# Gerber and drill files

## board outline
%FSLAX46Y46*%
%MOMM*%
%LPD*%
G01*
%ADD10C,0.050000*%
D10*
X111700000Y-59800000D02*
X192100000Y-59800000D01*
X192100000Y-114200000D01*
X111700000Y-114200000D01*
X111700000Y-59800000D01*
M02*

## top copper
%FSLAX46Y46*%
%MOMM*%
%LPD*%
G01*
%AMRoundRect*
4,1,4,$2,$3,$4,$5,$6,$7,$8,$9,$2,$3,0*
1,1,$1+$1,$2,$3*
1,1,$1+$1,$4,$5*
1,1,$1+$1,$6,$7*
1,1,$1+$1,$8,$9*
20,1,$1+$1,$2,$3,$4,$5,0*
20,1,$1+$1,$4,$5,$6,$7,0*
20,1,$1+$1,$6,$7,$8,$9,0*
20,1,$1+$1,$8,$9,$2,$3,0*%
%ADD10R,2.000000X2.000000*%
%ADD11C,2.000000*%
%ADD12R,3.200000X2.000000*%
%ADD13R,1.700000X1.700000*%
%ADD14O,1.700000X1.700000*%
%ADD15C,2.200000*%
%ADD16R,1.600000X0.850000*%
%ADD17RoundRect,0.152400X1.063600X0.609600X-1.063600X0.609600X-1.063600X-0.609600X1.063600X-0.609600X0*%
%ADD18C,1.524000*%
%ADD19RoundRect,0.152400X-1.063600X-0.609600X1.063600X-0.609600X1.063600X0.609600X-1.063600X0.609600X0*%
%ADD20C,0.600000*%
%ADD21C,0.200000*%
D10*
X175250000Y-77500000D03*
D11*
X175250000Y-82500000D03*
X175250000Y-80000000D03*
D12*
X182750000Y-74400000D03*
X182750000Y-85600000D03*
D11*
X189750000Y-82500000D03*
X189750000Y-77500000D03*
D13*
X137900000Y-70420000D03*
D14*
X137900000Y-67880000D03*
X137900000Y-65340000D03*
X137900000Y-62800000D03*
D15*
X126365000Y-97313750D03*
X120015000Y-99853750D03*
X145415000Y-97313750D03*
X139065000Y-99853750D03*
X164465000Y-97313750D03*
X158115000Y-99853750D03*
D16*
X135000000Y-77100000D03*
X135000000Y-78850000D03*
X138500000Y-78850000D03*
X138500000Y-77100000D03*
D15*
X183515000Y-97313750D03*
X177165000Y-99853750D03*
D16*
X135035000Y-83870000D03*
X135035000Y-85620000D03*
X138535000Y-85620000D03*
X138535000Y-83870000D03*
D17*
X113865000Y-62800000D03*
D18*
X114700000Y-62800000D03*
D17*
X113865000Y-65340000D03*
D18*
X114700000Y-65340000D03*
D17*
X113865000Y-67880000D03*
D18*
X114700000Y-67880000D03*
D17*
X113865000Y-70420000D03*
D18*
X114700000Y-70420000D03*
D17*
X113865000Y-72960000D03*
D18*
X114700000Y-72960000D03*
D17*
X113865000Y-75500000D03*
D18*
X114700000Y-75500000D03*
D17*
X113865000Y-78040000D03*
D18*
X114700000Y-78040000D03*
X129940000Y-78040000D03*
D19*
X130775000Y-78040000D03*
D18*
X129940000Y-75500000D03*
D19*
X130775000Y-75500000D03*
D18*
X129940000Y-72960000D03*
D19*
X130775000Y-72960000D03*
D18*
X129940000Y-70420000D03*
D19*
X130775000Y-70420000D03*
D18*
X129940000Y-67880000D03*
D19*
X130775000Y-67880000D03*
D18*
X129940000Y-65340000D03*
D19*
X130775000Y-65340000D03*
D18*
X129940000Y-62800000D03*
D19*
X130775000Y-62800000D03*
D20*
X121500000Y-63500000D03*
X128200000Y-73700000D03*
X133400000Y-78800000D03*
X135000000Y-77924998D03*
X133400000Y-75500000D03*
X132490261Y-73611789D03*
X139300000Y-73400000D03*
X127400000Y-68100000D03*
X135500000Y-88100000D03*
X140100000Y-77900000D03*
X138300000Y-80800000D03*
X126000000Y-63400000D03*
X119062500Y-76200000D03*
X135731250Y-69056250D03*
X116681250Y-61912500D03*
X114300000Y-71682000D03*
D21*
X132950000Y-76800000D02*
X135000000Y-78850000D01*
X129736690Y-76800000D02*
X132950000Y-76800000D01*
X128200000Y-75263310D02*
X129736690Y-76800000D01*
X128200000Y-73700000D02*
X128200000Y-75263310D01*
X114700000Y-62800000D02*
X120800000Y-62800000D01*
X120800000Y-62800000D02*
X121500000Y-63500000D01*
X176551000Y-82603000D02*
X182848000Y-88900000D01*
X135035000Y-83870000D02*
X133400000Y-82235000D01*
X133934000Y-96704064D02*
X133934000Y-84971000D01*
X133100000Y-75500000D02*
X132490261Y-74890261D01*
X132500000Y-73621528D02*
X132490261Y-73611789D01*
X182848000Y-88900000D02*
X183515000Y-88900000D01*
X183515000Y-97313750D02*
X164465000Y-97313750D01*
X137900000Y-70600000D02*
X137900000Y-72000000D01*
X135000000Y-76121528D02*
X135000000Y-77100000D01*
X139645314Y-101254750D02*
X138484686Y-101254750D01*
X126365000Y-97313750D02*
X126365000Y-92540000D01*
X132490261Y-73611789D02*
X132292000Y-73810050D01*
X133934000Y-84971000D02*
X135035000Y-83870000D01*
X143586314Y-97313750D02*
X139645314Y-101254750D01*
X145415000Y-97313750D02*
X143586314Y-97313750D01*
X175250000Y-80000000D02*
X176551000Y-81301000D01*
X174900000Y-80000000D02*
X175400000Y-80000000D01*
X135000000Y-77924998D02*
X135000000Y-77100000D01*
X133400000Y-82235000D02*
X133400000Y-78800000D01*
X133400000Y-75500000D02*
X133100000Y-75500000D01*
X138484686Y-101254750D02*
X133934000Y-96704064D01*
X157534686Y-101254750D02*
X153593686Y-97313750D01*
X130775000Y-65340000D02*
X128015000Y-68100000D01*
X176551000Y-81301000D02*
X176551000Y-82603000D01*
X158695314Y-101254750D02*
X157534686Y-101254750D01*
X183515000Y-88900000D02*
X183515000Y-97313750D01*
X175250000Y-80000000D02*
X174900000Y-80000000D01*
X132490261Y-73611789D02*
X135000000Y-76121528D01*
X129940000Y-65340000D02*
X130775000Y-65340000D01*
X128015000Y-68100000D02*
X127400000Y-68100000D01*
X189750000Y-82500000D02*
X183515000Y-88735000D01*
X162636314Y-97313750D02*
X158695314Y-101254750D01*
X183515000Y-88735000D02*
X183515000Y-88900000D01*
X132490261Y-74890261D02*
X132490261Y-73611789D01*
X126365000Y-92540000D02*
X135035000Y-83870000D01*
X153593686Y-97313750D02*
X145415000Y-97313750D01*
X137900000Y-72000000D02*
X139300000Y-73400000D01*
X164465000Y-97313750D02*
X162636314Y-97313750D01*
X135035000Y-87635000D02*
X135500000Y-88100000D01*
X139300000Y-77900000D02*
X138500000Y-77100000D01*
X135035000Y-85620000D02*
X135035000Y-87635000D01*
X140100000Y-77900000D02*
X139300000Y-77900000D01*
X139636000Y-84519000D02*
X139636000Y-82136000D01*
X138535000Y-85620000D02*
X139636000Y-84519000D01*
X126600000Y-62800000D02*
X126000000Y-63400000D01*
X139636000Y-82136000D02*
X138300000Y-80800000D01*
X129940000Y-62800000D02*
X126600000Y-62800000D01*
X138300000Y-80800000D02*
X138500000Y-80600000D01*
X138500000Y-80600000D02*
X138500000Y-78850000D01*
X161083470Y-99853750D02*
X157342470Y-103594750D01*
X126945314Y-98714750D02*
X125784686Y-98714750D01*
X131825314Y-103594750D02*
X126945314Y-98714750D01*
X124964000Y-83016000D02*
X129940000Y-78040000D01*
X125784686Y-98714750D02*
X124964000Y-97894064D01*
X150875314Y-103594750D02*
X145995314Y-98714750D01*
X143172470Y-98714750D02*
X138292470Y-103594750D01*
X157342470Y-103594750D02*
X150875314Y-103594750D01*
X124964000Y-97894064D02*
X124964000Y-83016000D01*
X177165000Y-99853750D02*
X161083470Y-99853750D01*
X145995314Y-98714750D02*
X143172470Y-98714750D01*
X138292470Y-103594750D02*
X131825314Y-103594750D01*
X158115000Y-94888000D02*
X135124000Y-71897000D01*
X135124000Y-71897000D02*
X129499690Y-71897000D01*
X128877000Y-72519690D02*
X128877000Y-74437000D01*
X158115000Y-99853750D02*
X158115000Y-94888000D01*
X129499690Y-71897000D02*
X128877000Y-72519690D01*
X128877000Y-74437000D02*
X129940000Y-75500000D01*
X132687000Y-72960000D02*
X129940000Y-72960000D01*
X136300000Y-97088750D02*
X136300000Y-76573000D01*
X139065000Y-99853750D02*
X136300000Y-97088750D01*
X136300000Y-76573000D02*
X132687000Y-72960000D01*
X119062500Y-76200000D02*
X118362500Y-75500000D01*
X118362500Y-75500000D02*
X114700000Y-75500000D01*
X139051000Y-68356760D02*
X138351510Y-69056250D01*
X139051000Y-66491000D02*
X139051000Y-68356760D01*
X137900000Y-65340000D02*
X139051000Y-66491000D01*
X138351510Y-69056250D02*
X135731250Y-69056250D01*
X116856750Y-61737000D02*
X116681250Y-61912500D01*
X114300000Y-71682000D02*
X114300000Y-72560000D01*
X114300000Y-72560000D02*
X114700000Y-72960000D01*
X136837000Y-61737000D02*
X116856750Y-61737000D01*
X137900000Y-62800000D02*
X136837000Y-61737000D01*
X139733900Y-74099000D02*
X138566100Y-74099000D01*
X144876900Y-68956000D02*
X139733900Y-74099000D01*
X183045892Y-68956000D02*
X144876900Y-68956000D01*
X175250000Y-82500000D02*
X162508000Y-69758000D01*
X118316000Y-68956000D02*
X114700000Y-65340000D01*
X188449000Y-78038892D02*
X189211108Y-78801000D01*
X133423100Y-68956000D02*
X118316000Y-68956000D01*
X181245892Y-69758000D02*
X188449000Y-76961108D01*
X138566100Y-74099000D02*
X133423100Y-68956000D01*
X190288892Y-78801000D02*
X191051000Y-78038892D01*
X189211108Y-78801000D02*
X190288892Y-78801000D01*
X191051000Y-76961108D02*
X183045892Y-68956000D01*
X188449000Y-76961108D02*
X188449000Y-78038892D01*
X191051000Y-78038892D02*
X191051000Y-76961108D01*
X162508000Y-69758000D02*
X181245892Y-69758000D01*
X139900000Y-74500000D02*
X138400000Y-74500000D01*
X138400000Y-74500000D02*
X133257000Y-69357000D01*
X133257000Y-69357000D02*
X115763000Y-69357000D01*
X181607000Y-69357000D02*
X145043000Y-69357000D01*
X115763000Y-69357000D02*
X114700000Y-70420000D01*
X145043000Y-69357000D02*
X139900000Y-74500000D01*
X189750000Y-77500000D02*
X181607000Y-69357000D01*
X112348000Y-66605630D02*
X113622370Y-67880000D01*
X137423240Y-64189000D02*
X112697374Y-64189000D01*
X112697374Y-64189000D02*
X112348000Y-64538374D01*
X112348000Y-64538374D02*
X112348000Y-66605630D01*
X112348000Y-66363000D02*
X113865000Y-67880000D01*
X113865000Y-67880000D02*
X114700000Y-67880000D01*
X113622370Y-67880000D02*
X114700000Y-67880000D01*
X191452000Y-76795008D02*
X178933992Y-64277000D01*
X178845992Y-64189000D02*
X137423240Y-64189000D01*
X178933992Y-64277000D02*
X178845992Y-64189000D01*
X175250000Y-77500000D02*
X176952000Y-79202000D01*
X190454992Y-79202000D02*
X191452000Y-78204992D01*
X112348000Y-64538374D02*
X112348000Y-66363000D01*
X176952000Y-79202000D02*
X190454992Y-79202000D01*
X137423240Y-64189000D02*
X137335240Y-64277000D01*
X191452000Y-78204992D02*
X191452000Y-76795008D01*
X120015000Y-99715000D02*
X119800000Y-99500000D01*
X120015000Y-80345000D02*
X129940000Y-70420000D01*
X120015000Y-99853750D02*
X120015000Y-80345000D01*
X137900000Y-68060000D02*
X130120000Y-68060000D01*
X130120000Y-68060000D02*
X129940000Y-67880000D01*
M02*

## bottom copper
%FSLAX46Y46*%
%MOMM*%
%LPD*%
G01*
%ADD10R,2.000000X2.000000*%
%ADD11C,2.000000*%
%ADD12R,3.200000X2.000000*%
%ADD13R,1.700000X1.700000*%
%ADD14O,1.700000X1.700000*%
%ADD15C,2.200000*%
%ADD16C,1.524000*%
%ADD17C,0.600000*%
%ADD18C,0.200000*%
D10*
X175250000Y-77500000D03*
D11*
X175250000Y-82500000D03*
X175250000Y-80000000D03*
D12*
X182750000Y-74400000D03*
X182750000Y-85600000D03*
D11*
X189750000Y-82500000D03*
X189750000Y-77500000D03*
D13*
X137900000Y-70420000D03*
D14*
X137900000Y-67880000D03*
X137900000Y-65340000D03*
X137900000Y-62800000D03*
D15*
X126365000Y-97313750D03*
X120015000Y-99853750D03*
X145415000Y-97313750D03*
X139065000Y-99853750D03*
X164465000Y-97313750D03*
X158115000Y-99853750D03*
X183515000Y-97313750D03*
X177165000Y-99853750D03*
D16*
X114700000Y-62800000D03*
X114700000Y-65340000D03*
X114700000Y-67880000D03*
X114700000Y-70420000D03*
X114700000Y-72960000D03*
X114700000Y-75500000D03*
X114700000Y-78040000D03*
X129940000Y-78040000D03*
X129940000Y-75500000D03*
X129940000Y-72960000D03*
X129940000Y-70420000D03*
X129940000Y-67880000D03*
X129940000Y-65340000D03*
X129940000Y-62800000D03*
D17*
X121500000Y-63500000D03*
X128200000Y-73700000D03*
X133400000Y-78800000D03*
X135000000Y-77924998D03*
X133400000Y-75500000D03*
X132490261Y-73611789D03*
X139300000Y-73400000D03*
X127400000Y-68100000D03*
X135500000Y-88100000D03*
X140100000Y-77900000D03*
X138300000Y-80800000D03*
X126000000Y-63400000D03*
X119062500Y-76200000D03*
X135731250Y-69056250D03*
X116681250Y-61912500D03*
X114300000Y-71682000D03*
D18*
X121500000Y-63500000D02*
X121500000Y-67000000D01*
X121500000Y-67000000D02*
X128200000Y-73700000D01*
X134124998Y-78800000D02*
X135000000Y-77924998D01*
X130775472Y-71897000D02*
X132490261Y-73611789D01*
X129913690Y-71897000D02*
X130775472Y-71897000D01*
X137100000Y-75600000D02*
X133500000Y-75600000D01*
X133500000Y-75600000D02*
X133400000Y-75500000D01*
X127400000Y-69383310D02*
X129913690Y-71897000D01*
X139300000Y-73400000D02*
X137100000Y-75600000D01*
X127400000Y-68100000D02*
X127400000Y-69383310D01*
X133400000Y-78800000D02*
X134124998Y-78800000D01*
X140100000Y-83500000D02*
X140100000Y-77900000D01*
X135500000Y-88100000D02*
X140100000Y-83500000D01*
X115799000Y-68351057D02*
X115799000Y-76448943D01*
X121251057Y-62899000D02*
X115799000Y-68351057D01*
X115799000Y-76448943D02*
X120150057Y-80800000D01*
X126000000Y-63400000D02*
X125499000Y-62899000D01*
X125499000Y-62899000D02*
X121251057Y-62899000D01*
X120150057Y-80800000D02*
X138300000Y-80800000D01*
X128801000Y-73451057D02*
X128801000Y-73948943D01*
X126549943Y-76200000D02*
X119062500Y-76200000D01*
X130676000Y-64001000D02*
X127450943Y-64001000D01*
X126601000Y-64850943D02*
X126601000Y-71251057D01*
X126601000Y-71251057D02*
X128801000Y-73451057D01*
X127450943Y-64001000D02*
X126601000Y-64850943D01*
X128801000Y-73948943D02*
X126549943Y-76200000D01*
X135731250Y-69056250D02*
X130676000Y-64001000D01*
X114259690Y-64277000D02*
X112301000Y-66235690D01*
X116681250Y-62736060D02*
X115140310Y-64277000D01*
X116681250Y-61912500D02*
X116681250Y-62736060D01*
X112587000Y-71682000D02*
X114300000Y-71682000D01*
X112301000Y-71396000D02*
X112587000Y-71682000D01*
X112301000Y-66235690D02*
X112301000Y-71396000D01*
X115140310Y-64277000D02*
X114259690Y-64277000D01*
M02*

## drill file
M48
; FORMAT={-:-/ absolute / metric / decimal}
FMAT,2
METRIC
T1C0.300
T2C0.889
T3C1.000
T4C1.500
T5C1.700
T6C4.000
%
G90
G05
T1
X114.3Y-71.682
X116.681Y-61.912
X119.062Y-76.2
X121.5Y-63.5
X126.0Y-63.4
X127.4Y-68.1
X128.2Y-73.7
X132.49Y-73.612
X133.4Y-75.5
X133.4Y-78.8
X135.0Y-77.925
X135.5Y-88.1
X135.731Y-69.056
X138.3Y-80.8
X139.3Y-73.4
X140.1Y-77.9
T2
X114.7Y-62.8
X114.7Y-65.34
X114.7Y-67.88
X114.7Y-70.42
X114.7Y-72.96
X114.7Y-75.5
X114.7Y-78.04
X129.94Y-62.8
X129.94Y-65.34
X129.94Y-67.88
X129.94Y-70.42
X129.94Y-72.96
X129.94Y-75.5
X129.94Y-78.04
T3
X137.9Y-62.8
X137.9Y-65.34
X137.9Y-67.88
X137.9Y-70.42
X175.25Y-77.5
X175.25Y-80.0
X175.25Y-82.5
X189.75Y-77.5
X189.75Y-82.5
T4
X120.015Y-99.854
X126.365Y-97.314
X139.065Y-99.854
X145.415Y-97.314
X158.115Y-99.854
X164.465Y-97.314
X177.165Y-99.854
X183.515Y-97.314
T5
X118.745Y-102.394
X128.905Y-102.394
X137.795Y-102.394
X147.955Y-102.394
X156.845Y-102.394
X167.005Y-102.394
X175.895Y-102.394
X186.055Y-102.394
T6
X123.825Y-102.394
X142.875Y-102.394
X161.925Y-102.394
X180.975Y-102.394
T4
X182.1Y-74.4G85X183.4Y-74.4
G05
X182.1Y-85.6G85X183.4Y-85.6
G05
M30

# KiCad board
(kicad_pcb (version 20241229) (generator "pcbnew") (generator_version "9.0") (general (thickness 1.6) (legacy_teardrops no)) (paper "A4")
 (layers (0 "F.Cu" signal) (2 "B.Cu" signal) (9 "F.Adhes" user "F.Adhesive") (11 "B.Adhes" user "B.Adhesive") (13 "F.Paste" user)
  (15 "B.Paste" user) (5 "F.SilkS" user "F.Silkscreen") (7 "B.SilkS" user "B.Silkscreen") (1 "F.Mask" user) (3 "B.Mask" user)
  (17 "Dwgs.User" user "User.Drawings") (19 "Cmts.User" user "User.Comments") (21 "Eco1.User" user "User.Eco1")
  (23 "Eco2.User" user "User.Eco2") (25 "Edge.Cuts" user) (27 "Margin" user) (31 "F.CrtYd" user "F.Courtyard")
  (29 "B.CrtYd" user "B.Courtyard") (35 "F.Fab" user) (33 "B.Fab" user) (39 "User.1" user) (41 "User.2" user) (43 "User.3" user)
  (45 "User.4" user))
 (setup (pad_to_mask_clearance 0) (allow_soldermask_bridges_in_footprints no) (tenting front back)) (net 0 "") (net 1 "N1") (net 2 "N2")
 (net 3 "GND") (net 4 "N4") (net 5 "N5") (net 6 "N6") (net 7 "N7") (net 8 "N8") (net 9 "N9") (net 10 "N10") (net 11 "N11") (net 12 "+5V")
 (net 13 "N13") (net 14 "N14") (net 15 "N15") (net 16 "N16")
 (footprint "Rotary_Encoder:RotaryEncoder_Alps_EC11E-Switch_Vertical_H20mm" (layer "F.Cu") (at 175.25 77.5)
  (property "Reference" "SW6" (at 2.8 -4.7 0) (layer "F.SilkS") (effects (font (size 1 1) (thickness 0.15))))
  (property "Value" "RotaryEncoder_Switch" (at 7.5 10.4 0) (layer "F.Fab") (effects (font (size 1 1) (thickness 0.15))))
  (pad "A" thru_hole rect (at 0 0) (size 2 2) (drill 1) (layers "*.Cu" "*.Mask") (remove_unused_layers no) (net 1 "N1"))
  (pad "B" thru_hole circle (at 0 5) (size 2 2) (drill 1) (layers "*.Cu" "*.Mask") (remove_unused_layers no) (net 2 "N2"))
  (pad "C" thru_hole circle (at 0 2.5) (size 2 2) (drill 1) (layers "*.Cu" "*.Mask") (remove_unused_layers no) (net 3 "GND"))
  (pad "MP" thru_hole rect (at 7.5 -3.1) (size 3.2 2) (drill oval 2.8 1.5) (layers "*.Cu" "*.Mask") (remove_unused_layers no))
  (pad "MP" thru_hole rect (at 7.5 8.1) (size 3.2 2) (drill oval 2.8 1.5) (layers "*.Cu" "*.Mask") (remove_unused_layers no))
  (pad "S1" thru_hole circle (at 14.5 5) (size 2 2) (drill 1) (layers "*.Cu" "*.Mask") (remove_unused_layers no) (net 3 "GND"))
  (pad "S2" thru_hole circle (at 14.5 0) (size 2 2) (drill 1) (layers "*.Cu" "*.Mask") (remove_unused_layers no) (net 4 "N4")))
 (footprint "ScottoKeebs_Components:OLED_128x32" (layer "F.Cu") (at 136.3 60.62)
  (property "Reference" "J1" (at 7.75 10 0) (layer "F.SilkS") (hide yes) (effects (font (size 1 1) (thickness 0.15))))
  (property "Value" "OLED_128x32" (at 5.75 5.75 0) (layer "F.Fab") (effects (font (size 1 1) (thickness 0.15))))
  (pad "1" thru_hole rect (at 1.6 9.8 180) (size 1.7 1.7) (drill 1) (layers "*.Cu" "*.Mask") (remove_unused_layers no) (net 3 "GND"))
  (pad "2" thru_hole oval (at 1.6 7.26 180) (size 1.7 1.7) (drill 1) (layers "*.Cu" "*.Mask") (remove_unused_layers no) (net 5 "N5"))
  (pad "3" thru_hole oval (at 1.6 4.72 180) (size 1.7 1.7) (drill 1) (layers "*.Cu" "*.Mask") (remove_unused_layers no) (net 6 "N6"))
  (pad "4" thru_hole oval (at 1.6 2.18 180) (size 1.7 1.7) (drill 1) (layers "*.Cu" "*.Mask") (remove_unused_layers no) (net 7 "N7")))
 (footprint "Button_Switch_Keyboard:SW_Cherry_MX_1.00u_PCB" (layer "F.Cu") (at 126.365 97.31375)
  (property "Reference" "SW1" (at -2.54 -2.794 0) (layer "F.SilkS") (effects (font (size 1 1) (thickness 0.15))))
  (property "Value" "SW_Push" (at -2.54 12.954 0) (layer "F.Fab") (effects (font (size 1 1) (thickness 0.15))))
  (pad "" np_thru_hole circle (at -7.62 5.08) (size 1.7 1.7) (drill 1.7) (layers "*.Cu" "*.Mask"))
  (pad "" np_thru_hole circle (at -2.54 5.08) (size 4 4) (drill 4) (layers "*.Cu" "*.Mask"))
  (pad "" np_thru_hole circle (at 2.54 5.08) (size 1.7 1.7) (drill 1.7) (layers "*.Cu" "*.Mask"))
  (pad "1" thru_hole circle (at 0 0) (size 2.2 2.2) (drill 1.5) (layers "*.Cu" "*.Mask") (remove_unused_layers no) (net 3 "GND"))
  (pad "2" thru_hole circle (at -6.35 2.54) (size 2.2 2.2) (drill 1.5) (layers "*.Cu" "*.Mask") (remove_unused_layers no) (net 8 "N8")))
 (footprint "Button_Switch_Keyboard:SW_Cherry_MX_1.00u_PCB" (layer "F.Cu") (at 145.415 97.31375)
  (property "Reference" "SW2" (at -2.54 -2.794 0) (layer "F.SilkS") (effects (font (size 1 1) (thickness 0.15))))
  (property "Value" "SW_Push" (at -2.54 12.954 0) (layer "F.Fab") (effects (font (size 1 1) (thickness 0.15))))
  (pad "" np_thru_hole circle (at -7.62 5.08) (size 1.7 1.7) (drill 1.7) (layers "*.Cu" "*.Mask"))
  (pad "" np_thru_hole circle (at -2.54 5.08) (size 4 4) (drill 4) (layers "*.Cu" "*.Mask"))
  (pad "" np_thru_hole circle (at 2.54 5.08) (size 1.7 1.7) (drill 1.7) (layers "*.Cu" "*.Mask"))
  (pad "1" thru_hole circle (at 0 0) (size 2.2 2.2) (drill 1.5) (layers "*.Cu" "*.Mask") (remove_unused_layers no) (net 3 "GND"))
  (pad "2" thru_hole circle (at -6.35 2.54) (size 2.2 2.2) (drill 1.5) (layers "*.Cu" "*.Mask") (remove_unused_layers no) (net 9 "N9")))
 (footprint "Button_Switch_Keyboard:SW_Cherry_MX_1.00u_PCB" (layer "F.Cu") (at 164.465 97.31375)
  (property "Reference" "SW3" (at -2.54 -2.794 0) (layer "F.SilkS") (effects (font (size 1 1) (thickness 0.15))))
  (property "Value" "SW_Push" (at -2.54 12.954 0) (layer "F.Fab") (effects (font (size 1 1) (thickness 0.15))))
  (pad "" np_thru_hole circle (at -7.62 5.08) (size 1.7 1.7) (drill 1.7) (layers "*.Cu" "*.Mask"))
  (pad "" np_thru_hole circle (at -2.54 5.08) (size 4 4) (drill 4) (layers "*.Cu" "*.Mask"))
  (pad "" np_thru_hole circle (at 2.54 5.08) (size 1.7 1.7) (drill 1.7) (layers "*.Cu" "*.Mask"))
  (pad "1" thru_hole circle (at 0 0) (size 2.2 2.2) (drill 1.5) (layers "*.Cu" "*.Mask") (remove_unused_layers no) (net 3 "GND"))
  (pad "2" thru_hole circle (at -6.35 2.54) (size 2.2 2.2) (drill 1.5) (layers "*.Cu" "*.Mask") (remove_unused_layers no) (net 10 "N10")))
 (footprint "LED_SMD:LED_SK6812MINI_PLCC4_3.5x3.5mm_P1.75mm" (layer "F.Cu") (at 136.75 77.975)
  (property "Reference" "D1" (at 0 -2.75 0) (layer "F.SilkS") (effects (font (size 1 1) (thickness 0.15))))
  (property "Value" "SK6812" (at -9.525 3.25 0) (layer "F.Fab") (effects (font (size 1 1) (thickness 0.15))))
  (pad "1" smd rect (at -1.75 -0.875) (size 1.6 0.85) (layers "F.Cu" "F.Mask" "F.Paste") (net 3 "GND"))
  (pad "2" smd rect (at -1.75 0.875) (size 1.6 0.85) (layers "F.Cu" "F.Mask" "F.Paste") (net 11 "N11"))
  (pad "3" smd rect (at 1.75 0.875) (size 1.6 0.85) (layers "F.Cu" "F.Mask" "F.Paste") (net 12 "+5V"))
  (pad "4" smd rect (at 1.75 -0.875) (size 1.6 0.85) (layers "F.Cu" "F.Mask" "F.Paste") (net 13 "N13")))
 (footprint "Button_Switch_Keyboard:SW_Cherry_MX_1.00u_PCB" (layer "F.Cu") (at 183.515 97.31375)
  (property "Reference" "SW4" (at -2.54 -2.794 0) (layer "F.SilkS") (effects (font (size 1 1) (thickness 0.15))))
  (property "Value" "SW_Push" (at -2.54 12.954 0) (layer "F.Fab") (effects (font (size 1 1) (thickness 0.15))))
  (pad "" np_thru_hole circle (at -7.62 5.08) (size 1.7 1.7) (drill 1.7) (layers "*.Cu" "*.Mask"))
  (pad "" np_thru_hole circle (at -2.54 5.08) (size 4 4) (drill 4) (layers "*.Cu" "*.Mask"))
  (pad "" np_thru_hole circle (at 2.54 5.08) (size 1.7 1.7) (drill 1.7) (layers "*.Cu" "*.Mask"))
  (pad "1" thru_hole circle (at 0 0) (size 2.2 2.2) (drill 1.5) (layers "*.Cu" "*.Mask") (remove_unused_layers no) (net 3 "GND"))
  (pad "2" thru_hole circle (at -6.35 2.54) (size 2.2 2.2) (drill 1.5) (layers "*.Cu" "*.Mask") (remove_unused_layers no) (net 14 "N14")))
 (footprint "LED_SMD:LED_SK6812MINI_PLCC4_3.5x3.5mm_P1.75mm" (layer "F.Cu") (at 136.785 84.745)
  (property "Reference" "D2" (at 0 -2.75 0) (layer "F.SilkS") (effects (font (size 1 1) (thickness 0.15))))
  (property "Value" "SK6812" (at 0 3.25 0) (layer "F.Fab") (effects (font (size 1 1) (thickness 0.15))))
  (pad "1" smd rect (at -1.75 -0.875) (size 1.6 0.85) (layers "F.Cu" "F.Mask" "F.Paste") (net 3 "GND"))
  (pad "2" smd rect (at -1.75 0.875) (size 1.6 0.85) (layers "F.Cu" "F.Mask" "F.Paste") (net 13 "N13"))
  (pad "3" smd rect (at 1.75 0.875) (size 1.6 0.85) (layers "F.Cu" "F.Mask" "F.Paste") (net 12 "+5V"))
  (pad "4" smd rect (at 1.75 -0.875) (size 1.6 0.85) (layers "F.Cu" "F.Mask" "F.Paste") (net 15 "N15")))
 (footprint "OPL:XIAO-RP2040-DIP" (layer "F.Cu") (at 122.32 70.42)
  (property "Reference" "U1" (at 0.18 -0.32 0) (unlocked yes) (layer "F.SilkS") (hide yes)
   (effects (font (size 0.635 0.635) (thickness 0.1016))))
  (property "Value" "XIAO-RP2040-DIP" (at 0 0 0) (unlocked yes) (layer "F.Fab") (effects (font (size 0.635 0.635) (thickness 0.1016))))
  (pad "1" smd roundrect (at -8.455 -7.62 180) (size 2.432 1.524) (layers "F.Cu" "F.Mask") (roundrect_rratio 0.1) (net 11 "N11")
   (thermal_bridge_angle 45))
  (pad "1" thru_hole circle (at -7.62 -7.62 180) (size 1.524 1.524) (drill 0.889) (layers "*.Cu" "*.Mask") (remove_unused_layers no)
   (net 11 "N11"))
  (pad "2" smd roundrect (at -8.455 -5.08 180) (size 2.432 1.524) (layers "F.Cu" "F.Mask") (roundrect_rratio 0.1) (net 2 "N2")
   (thermal_bridge_angle 45))
  (pad "2" thru_hole circle (at -7.62 -5.08 180) (size 1.524 1.524) (drill 0.889) (layers "*.Cu" "*.Mask") (remove_unused_layers no)
   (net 2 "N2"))
  (pad "3" smd roundrect (at -8.455 -2.54 180) (size 2.432 1.524) (layers "F.Cu" "F.Mask") (roundrect_rratio 0.1) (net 1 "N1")
   (thermal_bridge_angle 45))
  (pad "3" thru_hole circle (at -7.62 -2.54 180) (size 1.524 1.524) (drill 0.889) (layers "*.Cu" "*.Mask") (remove_unused_layers no)
   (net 1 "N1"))
  (pad "4" smd roundrect (at -8.455 0 180) (size 2.432 1.524) (layers "F.Cu" "F.Mask") (roundrect_rratio 0.1) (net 4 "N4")
   (thermal_bridge_angle 45))
  (pad "4" thru_hole circle (at -7.62 0 180) (size 1.524 1.524) (drill 0.889) (layers "*.Cu" "*.Mask") (remove_unused_layers no)
   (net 4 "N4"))
  (pad "5" smd roundrect (at -8.455 2.54 180) (size 2.432 1.524) (layers "F.Cu" "F.Mask") (roundrect_rratio 0.1) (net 7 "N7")
   (thermal_bridge_angle 45))
  (pad "5" thru_hole circle (at -7.62 2.54 180) (size 1.524 1.524) (drill 0.889) (layers "*.Cu" "*.Mask") (remove_unused_layers no)
   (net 7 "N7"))
  (pad "6" smd roundrect (at -8.455 5.08 180) (size 2.432 1.524) (layers "F.Cu" "F.Mask") (roundrect_rratio 0.1) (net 6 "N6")
   (thermal_bridge_angle 45))
  (pad "6" thru_hole circle (at -7.62 5.08 180) (size 1.524 1.524) (drill 0.889) (layers "*.Cu" "*.Mask") (remove_unused_layers no)
   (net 6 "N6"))
  (pad "7" smd roundrect (at -8.455 7.62 180) (size 2.432 1.524) (layers "F.Cu" "F.Mask") (roundrect_rratio 0.1) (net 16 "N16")
   (thermal_bridge_angle 45))
  (pad "7" thru_hole circle (at -7.62 7.62 180) (size 1.524 1.524) (drill 0.889) (layers "*.Cu" "*.Mask") (remove_unused_layers no)
   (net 16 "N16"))
  (pad "8" thru_hole circle (at 7.62 7.62) (size 1.524 1.524) (drill 0.889) (layers "*.Cu" "*.Mask") (remove_unused_layers no)
   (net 14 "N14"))
  (pad "8" smd roundrect (at 8.455 7.62) (size 2.432 1.524) (layers "F.Cu" "F.Mask") (roundrect_rratio 0.1) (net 14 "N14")
   (thermal_bridge_angle 45))
  (pad "9" thru_hole circle (at 7.62 5.08) (size 1.524 1.524) (drill 0.889) (layers "*.Cu" "*.Mask") (remove_unused_layers no)
   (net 10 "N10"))
  (pad "9" smd roundrect (at 8.455 5.08) (size 2.432 1.524) (layers "F.Cu" "F.Mask") (roundrect_rratio 0.1) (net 10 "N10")
   (thermal_bridge_angle 45))
  (pad "10" thru_hole circle (at 7.62 2.54) (size 1.524 1.524) (drill 0.889) (layers "*.Cu" "*.Mask") (remove_unused_layers no) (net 9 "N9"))
  (pad "10" smd roundrect (at 8.455 2.54) (size 2.432 1.524) (layers "F.Cu" "F.Mask") (roundrect_rratio 0.1) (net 9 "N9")
   (thermal_bridge_angle 45))
  (pad "11" thru_hole circle (at 7.62 0) (size 1.524 1.524) (drill 0.889) (layers "*.Cu" "*.Mask") (remove_unused_layers no) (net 8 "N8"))
  (pad "11" smd roundrect (at 8.455 0) (size 2.432 1.524) (layers "F.Cu" "F.Mask") (roundrect_rratio 0.1) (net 8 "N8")
   (thermal_bridge_angle 45))
  (pad "12" thru_hole circle (at 7.62 -2.54) (size 1.524 1.524) (drill 0.889) (layers "*.Cu" "*.Mask") (remove_unused_layers no)
   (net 5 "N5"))
  (pad "12" smd roundrect (at 8.455 -2.54) (size 2.432 1.524) (layers "F.Cu" "F.Mask") (roundrect_rratio 0.1) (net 5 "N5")
   (thermal_bridge_angle 45))
  (pad "13" thru_hole circle (at 7.62 -5.08) (size 1.524 1.524) (drill 0.889) (layers "*.Cu" "*.Mask") (remove_unused_layers no)
   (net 3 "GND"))
  (pad "13" smd roundrect (at 8.455 -5.08) (size 2.432 1.524) (layers "F.Cu" "F.Mask") (roundrect_rratio 0.1) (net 3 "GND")
   (thermal_bridge_angle 45))
  (pad "14" thru_hole circle (at 7.62 -7.62) (size 1.524 1.524) (drill 0.889) (layers "*.Cu" "*.Mask") (remove_unused_layers no)
   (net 12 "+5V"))
  (pad "14" smd roundrect (at 8.455 -7.62) (size 2.432 1.524) (layers "F.Cu" "F.Mask") (roundrect_rratio 0.1) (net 12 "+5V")
   (thermal_bridge_angle 45)))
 (gr_rect (start 111.7 59.8) (end 192.1 114.2) (stroke (width 0.05) (type default)) (fill no) (layer "Edge.Cuts"))
 (segment (start 132.95 76.8) (end 135 78.85) (width 0.2) (layer "F.Cu") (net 11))
 (segment (start 129.73669 76.8) (end 132.95 76.8) (width 0.2) (layer "F.Cu") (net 11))
 (segment (start 128.2 75.26331) (end 129.73669 76.8) (width 0.2) (layer "F.Cu") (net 11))
 (segment (start 128.2 73.7) (end 128.2 75.26331) (width 0.2) (layer "F.Cu") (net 11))
 (segment (start 114.7 62.8) (end 120.8 62.8) (width 0.2) (layer "F.Cu") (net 11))
 (segment (start 120.8 62.8) (end 121.5 63.5) (width 0.2) (layer "F.Cu") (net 11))
 (via (at 121.5 63.5) (size 0.6) (drill 0.3) (layers "F.Cu" "B.Cu") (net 11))
 (via (at 128.2 73.7) (size 0.6) (drill 0.3) (layers "F.Cu" "B.Cu") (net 11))
 (segment (start 121.5 63.5) (end 121.5 67) (width 0.2) (layer "B.Cu") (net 11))
 (segment (start 121.5 67) (end 128.2 73.7) (width 0.2) (layer "B.Cu") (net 11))
 (segment (start 176.551 82.603) (end 182.848 88.9) (width 0.2) (layer "F.Cu") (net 3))
 (segment (start 135.035 83.87) (end 133.4 82.235) (width 0.2) (layer "F.Cu") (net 3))
 (segment (start 133.934 96.704064) (end 133.934 84.971) (width 0.2) (layer "F.Cu") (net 3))
 (segment (start 133.1 75.5) (end 132.490261 74.890261) (width 0.2) (layer "F.Cu") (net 3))
 (segment (start 132.5 73.621528) (end 132.490261 73.611789) (width 0.2) (layer "F.Cu") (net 3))
 (segment (start 182.848 88.9) (end 183.515 88.9) (width 0.2) (layer "F.Cu") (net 3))
 (segment (start 183.515 97.31375) (end 164.465 97.31375) (width 0.2) (layer "F.Cu") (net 3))
 (segment (start 137.9 70.6) (end 137.9 72) (width 0.2) (layer "F.Cu") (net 3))
 (segment (start 135 76.121528) (end 135 77.1) (width 0.2) (layer "F.Cu") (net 3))
 (segment (start 139.645314 101.25475) (end 138.484686 101.25475) (width 0.2) (layer "F.Cu") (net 3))
 (segment (start 126.365 97.31375) (end 126.365 92.54) (width 0.2) (layer "F.Cu") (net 3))
 (segment (start 132.490261 73.611789) (end 132.292 73.81005) (width 0.2) (layer "F.Cu") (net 3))
 (segment (start 133.934 84.971) (end 135.035 83.87) (width 0.2) (layer "F.Cu") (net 3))
 (segment (start 143.586314 97.31375) (end 139.645314 101.25475) (width 0.2) (layer "F.Cu") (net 3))
 (segment (start 145.415 97.31375) (end 143.586314 97.31375) (width 0.2) (layer "F.Cu") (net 3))
 (segment (start 175.25 80) (end 176.551 81.301) (width 0.2) (layer "F.Cu") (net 3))
 (segment (start 174.9 80) (end 175.4 80) (width 0.2) (layer "F.Cu") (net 3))
 (segment (start 135 77.924998) (end 135 77.1) (width 0.2) (layer "F.Cu") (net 3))
 (segment (start 133.4 82.235) (end 133.4 78.8) (width 0.2) (layer "F.Cu") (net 3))
 (segment (start 133.4 75.5) (end 133.1 75.5) (width 0.2) (layer "F.Cu") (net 3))
 (segment (start 138.484686 101.25475) (end 133.934 96.704064) (width 0.2) (layer "F.Cu") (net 3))
 (segment (start 157.534686 101.25475) (end 153.593686 97.31375) (width 0.2) (layer "F.Cu") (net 3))
 (segment (start 130.775 65.34) (end 128.015 68.1) (width 0.2) (layer "F.Cu") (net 3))
 (segment (start 176.551 81.301) (end 176.551 82.603) (width 0.2) (layer "F.Cu") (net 3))
 (segment (start 158.695314 101.25475) (end 157.534686 101.25475) (width 0.2) (layer "F.Cu") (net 3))
 (segment (start 183.515 88.9) (end 183.515 97.31375) (width 0.2) (layer "F.Cu") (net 3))
 (segment (start 175.25 80) (end 174.9 80) (width 0.2) (layer "F.Cu") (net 3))
 (segment (start 132.490261 73.611789) (end 135 76.121528) (width 0.2) (layer "F.Cu") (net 3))
 (segment (start 129.94 65.34) (end 130.775 65.34) (width 0.2) (layer "F.Cu") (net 3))
 (segment (start 128.015 68.1) (end 127.4 68.1) (width 0.2) (layer "F.Cu") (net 3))
 (segment (start 189.75 82.5) (end 183.515 88.735) (width 0.2) (layer "F.Cu") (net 3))
 (segment (start 162.636314 97.31375) (end 158.695314 101.25475) (width 0.2) (layer "F.Cu") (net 3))
 (segment (start 183.515 88.735) (end 183.515 88.9) (width 0.2) (layer "F.Cu") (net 3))
 (segment (start 132.490261 74.890261) (end 132.490261 73.611789) (width 0.2) (layer "F.Cu") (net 3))
 (segment (start 126.365 92.54) (end 135.035 83.87) (width 0.2) (layer "F.Cu") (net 3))
 (segment (start 153.593686 97.31375) (end 145.415 97.31375) (width 0.2) (layer "F.Cu") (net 3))
 (segment (start 137.9 72) (end 139.3 73.4) (width 0.2) (layer "F.Cu") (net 3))
 (segment (start 164.465 97.31375) (end 162.636314 97.31375) (width 0.2) (layer "F.Cu") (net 3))
 (via (at 133.4 78.8) (size 0.6) (drill 0.3) (layers "F.Cu" "B.Cu") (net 3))
 (via (at 135 77.924998) (size 0.6) (drill 0.3) (layers "F.Cu" "B.Cu") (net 3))
 (via (at 133.4 75.5) (size 0.6) (drill 0.3) (layers "F.Cu" "B.Cu") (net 3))
 (via (at 132.490261 73.611789) (size 0.6) (drill 0.3) (layers "F.Cu" "B.Cu") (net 3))
 (via (at 139.3 73.4) (size 0.6) (drill 0.3) (layers "F.Cu" "B.Cu") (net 3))
 (via (at 127.4 68.1) (size 0.6) (drill 0.3) (layers "F.Cu" "B.Cu") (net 3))
 (segment (start 134.124998 78.8) (end 135 77.924998) (width 0.2) (layer "B.Cu") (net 3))
 (segment (start 130.775472 71.897) (end 132.490261 73.611789) (width 0.2) (layer "B.Cu") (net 3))
 (segment (start 129.91369 71.897) (end 130.775472 71.897) (width 0.2) (layer "B.Cu") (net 3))
 (segment (start 137.1 75.6) (end 133.5 75.6) (width 0.2) (layer "B.Cu") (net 3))
 (segment (start 133.5 75.6) (end 133.4 75.5) (width 0.2) (layer "B.Cu") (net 3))
 (segment (start 127.4 69.38331) (end 129.91369 71.897) (width 0.2) (layer "B.Cu") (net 3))
 (segment (start 139.3 73.4) (end 137.1 75.6) (width 0.2) (layer "B.Cu") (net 3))
 (segment (start 127.4 68.1) (end 127.4 69.38331) (width 0.2) (layer "B.Cu") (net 3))
 (segment (start 133.4 78.8) (end 134.124998 78.8) (width 0.2) (layer "B.Cu") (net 3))
 (segment (start 135.035 87.635) (end 135.5 88.1) (width 0.2) (layer "F.Cu") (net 13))
 (segment (start 139.3 77.9) (end 138.5 77.1) (width 0.2) (layer "F.Cu") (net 13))
 (segment (start 135.035 85.62) (end 135.035 87.635) (width 0.2) (layer "F.Cu") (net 13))
 (segment (start 140.1 77.9) (end 139.3 77.9) (width 0.2) (layer "F.Cu") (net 13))
 (via (at 135.5 88.1) (size 0.6) (drill 0.3) (layers "F.Cu" "B.Cu") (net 13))
 (via (at 140.1 77.9) (size 0.6) (drill 0.3) (layers "F.Cu" "B.Cu") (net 13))
 (segment (start 140.1 83.5) (end 140.1 77.9) (width 0.2) (layer "B.Cu") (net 13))
 (segment (start 135.5 88.1) (end 140.1 83.5) (width 0.2) (layer "B.Cu") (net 13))
 (segment (start 139.636 84.519) (end 139.636 82.136) (width 0.2) (layer "F.Cu") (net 12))
 (segment (start 138.535 85.62) (end 139.636 84.519) (width 0.2) (layer "F.Cu") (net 12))
 (segment (start 126.6 62.8) (end 126 63.4) (width 0.2) (layer "F.Cu") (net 12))
 (segment (start 139.636 82.136) (end 138.3 80.8) (width 0.2) (layer "F.Cu") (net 12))
 (segment (start 129.94 62.8) (end 126.6 62.8) (width 0.2) (layer "F.Cu") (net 12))
 (segment (start 138.3 80.8) (end 138.5 80.6) (width 0.2) (layer "F.Cu") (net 12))
 (segment (start 138.5 80.6) (end 138.5 78.85) (width 0.2) (layer "F.Cu") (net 12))
 (via (at 138.3 80.8) (size 0.6) (drill 0.3) (layers "F.Cu" "B.Cu") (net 12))
 (via (at 126 63.4) (size 0.6) (drill 0.3) (layers "F.Cu" "B.Cu") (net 12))
 (segment (start 115.799 68.351057) (end 115.799 76.448943) (width 0.2) (layer "B.Cu") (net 12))
 (segment (start 121.251057 62.899) (end 115.799 68.351057) (width 0.2) (layer "B.Cu") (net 12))
 (segment (start 115.799 76.448943) (end 120.150057 80.8) (width 0.2) (layer "B.Cu") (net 12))
 (segment (start 126 63.4) (end 125.499 62.899) (width 0.2) (layer "B.Cu") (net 12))
 (segment (start 125.499 62.899) (end 121.251057 62.899) (width 0.2) (layer "B.Cu") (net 12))
 (segment (start 120.150057 80.8) (end 138.3 80.8) (width 0.2) (layer "B.Cu") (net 12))
 (segment (start 161.08347 99.85375) (end 157.34247 103.59475) (width 0.2) (layer "F.Cu") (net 14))
 (segment (start 126.945314 98.71475) (end 125.784686 98.71475) (width 0.2) (layer "F.Cu") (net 14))
 (segment (start 131.825314 103.59475) (end 126.945314 98.71475) (width 0.2) (layer "F.Cu") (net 14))
 (segment (start 124.964 83.016) (end 129.94 78.04) (width 0.2) (layer "F.Cu") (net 14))
 (segment (start 125.784686 98.71475) (end 124.964 97.894064) (width 0.2) (layer "F.Cu") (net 14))
 (segment (start 150.875314 103.59475) (end 145.995314 98.71475) (width 0.2) (layer "F.Cu") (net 14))
 (segment (start 143.17247 98.71475) (end 138.29247 103.59475) (width 0.2) (layer "F.Cu") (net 14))
 (segment (start 157.34247 103.59475) (end 150.875314 103.59475) (width 0.2) (layer "F.Cu") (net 14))
 (segment (start 124.964 97.894064) (end 124.964 83.016) (width 0.2) (layer "F.Cu") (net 14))
 (segment (start 177.165 99.85375) (end 161.08347 99.85375) (width 0.2) (layer "F.Cu") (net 14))
 (segment (start 145.995314 98.71475) (end 143.17247 98.71475) (width 0.2) (layer "F.Cu") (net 14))
 (segment (start 138.29247 103.59475) (end 131.825314 103.59475) (width 0.2) (layer "F.Cu") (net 14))
 (segment (start 158.115 94.888) (end 135.124 71.897) (width 0.2) (layer "F.Cu") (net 10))
 (segment (start 135.124 71.897) (end 129.49969 71.897) (width 0.2) (layer "F.Cu") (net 10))
 (segment (start 128.877 72.51969) (end 128.877 74.437) (width 0.2) (layer "F.Cu") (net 10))
 (segment (start 158.115 99.85375) (end 158.115 94.888) (width 0.2) (layer "F.Cu") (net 10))
 (segment (start 129.49969 71.897) (end 128.877 72.51969) (width 0.2) (layer "F.Cu") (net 10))
 (segment (start 128.877 74.437) (end 129.94 75.5) (width 0.2) (layer "F.Cu") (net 10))
 (segment (start 132.687 72.96) (end 129.94 72.96) (width 0.2) (layer "F.Cu") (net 9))
 (segment (start 136.3 97.08875) (end 136.3 76.573) (width 0.2) (layer "F.Cu") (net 9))
 (segment (start 139.065 99.85375) (end 136.3 97.08875) (width 0.2) (layer "F.Cu") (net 9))
 (segment (start 136.3 76.573) (end 132.687 72.96) (width 0.2) (layer "F.Cu") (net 9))
 (segment (start 119.0625 76.2) (end 118.3625 75.5) (width 0.2) (layer "F.Cu") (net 6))
 (segment (start 118.3625 75.5) (end 114.7 75.5) (width 0.2) (layer "F.Cu") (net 6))
 (segment (start 139.051 68.35676) (end 138.35151 69.05625) (width 0.2) (layer "F.Cu") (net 6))
 (segment (start 139.051 66.491) (end 139.051 68.35676) (width 0.2) (layer "F.Cu") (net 6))
 (segment (start 137.9 65.34) (end 139.051 66.491) (width 0.2) (layer "F.Cu") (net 6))
 (segment (start 138.35151 69.05625) (end 135.73125 69.05625) (width 0.2) (layer "F.Cu") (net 6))
 (via (at 119.0625 76.2) (size 0.6) (drill 0.3) (layers "F.Cu" "B.Cu") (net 6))
 (via (at 135.73125 69.05625) (size 0.6) (drill 0.3) (layers "F.Cu" "B.Cu") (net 6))
 (segment (start 128.801 73.451057) (end 128.801 73.948943) (width 0.2) (layer "B.Cu") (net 6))
 (segment (start 126.549943 76.2) (end 119.0625 76.2) (width 0.2) (layer "B.Cu") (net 6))
 (segment (start 130.676 64.001) (end 127.450943 64.001) (width 0.2) (layer "B.Cu") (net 6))
 (segment (start 126.601 64.850943) (end 126.601 71.251057) (width 0.2) (layer "B.Cu") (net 6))
 (segment (start 126.601 71.251057) (end 128.801 73.451057) (width 0.2) (layer "B.Cu") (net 6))
 (segment (start 127.450943 64.001) (end 126.601 64.850943) (width 0.2) (layer "B.Cu") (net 6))
 (segment (start 128.801 73.948943) (end 126.549943 76.2) (width 0.2) (layer "B.Cu") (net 6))
 (segment (start 135.73125 69.05625) (end 130.676 64.001) (width 0.2) (layer "B.Cu") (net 6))
 (segment (start 116.85675 61.737) (end 116.68125 61.9125) (width 0.2) (layer "F.Cu") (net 7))
 (segment (start 114.3 71.682) (end 114.3 72.56) (width 0.2) (layer "F.Cu") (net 7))
 (segment (start 114.3 72.56) (end 114.7 72.96) (width 0.2) (layer "F.Cu") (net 7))
 (segment (start 136.837 61.737) (end 116.85675 61.737) (width 0.2) (layer "F.Cu") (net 7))
 (segment (start 137.9 62.8) (end 136.837 61.737) (width 0.2) (layer "F.Cu") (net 7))
 (via (at 116.68125 61.9125) (size 0.6) (drill 0.3) (layers "F.Cu" "B.Cu") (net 7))
 (via (at 114.3 71.682) (size 0.6) (drill 0.3) (layers "F.Cu" "B.Cu") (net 7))
 (segment (start 114.25969 64.277) (end 112.301 66.23569) (width 0.2) (layer "B.Cu") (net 7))
 (segment (start 116.68125 62.73606) (end 115.14031 64.277) (width 0.2) (layer "B.Cu") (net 7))
 (segment (start 116.68125 61.9125) (end 116.68125 62.73606) (width 0.2) (layer "B.Cu") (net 7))
 (segment (start 112.587 71.682) (end 114.3 71.682) (width 0.2) (layer "B.Cu") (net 7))
 (segment (start 112.301 71.396) (end 112.587 71.682) (width 0.2) (layer "B.Cu") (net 7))
 (segment (start 112.301 66.23569) (end 112.301 71.396) (width 0.2) (layer "B.Cu") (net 7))
 (segment (start 115.14031 64.277) (end 114.25969 64.277) (width 0.2) (layer "B.Cu") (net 7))
 (segment (start 139.7339 74.099) (end 138.5661 74.099) (width 0.2) (layer "F.Cu") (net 2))
 (segment (start 144.8769 68.956) (end 139.7339 74.099) (width 0.2) (layer "F.Cu") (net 2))
 (segment (start 183.045892 68.956) (end 144.8769 68.956) (width 0.2) (layer "F.Cu") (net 2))
 (segment (start 175.25 82.5) (end 162.508 69.758) (width 0.2) (layer "F.Cu") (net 2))
 (segment (start 118.316 68.956) (end 114.7 65.34) (width 0.2) (layer "F.Cu") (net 2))
 (segment (start 188.449 78.038892) (end 189.211108 78.801) (width 0.2) (layer "F.Cu") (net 2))
 (segment (start 133.4231 68.956) (end 118.316 68.956) (width 0.2) (layer "F.Cu") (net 2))
 (segment (start 181.245892 69.758) (end 188.449 76.961108) (width 0.2) (layer "F.Cu") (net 2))
 (segment (start 138.5661 74.099) (end 133.4231 68.956) (width 0.2) (layer "F.Cu") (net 2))
 (segment (start 190.288892 78.801) (end 191.051 78.038892) (width 0.2) (layer "F.Cu") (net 2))
 (segment (start 189.211108 78.801) (end 190.288892 78.801) (width 0.2) (layer "F.Cu") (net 2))
 (segment (start 191.051 76.961108) (end 183.045892 68.956) (width 0.2) (layer "F.Cu") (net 2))
 (segment (start 188.449 76.961108) (end 188.449 78.038892) (width 0.2) (layer "F.Cu") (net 2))
 (segment (start 191.051 78.038892) (end 191.051 76.961108) (width 0.2) (layer "F.Cu") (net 2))
 (segment (start 162.508 69.758) (end 181.245892 69.758) (width 0.2) (layer "F.Cu") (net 2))
 (segment (start 139.9 74.5) (end 138.4 74.5) (width 0.2) (layer "F.Cu") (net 4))
 (segment (start 138.4 74.5) (end 133.257 69.357) (width 0.2) (layer "F.Cu") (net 4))
 (segment (start 133.257 69.357) (end 115.763 69.357) (width 0.2) (layer "F.Cu") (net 4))
 (segment (start 181.607 69.357) (end 145.043 69.357) (width 0.2) (layer "F.Cu") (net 4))
 (segment (start 115.763 69.357) (end 114.7 70.42) (width 0.2) (layer "F.Cu") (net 4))
 (segment (start 145.043 69.357) (end 139.9 74.5) (width 0.2) (layer "F.Cu") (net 4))
 (segment (start 189.75 77.5) (end 181.607 69.357) (width 0.2) (layer "F.Cu") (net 4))
 (segment (start 112.348 66.60563) (end 113.62237 67.88) (width 0.2) (layer "F.Cu") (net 1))
 (segment (start 137.42324 64.189) (end 112.697374 64.189) (width 0.2) (layer "F.Cu") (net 1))
 (segment (start 112.697374 64.189) (end 112.348 64.538374) (width 0.2) (layer "F.Cu") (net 1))
 (segment (start 112.348 64.538374) (end 112.348 66.60563) (width 0.2) (layer "F.Cu") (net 1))
 (segment (start 112.348 66.363) (end 113.865 67.88) (width 0.2) (layer "F.Cu") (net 1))
 (segment (start 113.865 67.88) (end 114.7 67.88) (width 0.2) (layer "F.Cu") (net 1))
 (segment (start 113.62237 67.88) (end 114.7 67.88) (width 0.2) (layer "F.Cu") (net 1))
 (segment (start 191.452 76.795008) (end 178.933992 64.277) (width 0.2) (layer "F.Cu") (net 1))
 (segment (start 178.845992 64.189) (end 137.42324 64.189) (width 0.2) (layer "F.Cu") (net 1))
 (segment (start 178.933992 64.277) (end 178.845992 64.189) (width 0.2) (layer "F.Cu") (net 1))
 (segment (start 175.25 77.5) (end 176.952 79.202) (width 0.2) (layer "F.Cu") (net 1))
 (segment (start 190.454992 79.202) (end 191.452 78.204992) (width 0.2) (layer "F.Cu") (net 1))
 (segment (start 112.348 64.538374) (end 112.348 66.363) (width 0.2) (layer "F.Cu") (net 1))
 (segment (start 176.952 79.202) (end 190.454992 79.202) (width 0.2) (layer "F.Cu") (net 1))
 (segment (start 137.42324 64.189) (end 137.33524 64.277) (width 0.2) (layer "F.Cu") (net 1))
 (segment (start 191.452 78.204992) (end 191.452 76.795008) (width 0.2) (layer "F.Cu") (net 1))
 (segment (start 120.015 99.715) (end 119.8 99.5) (width 0.2) (layer "F.Cu") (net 8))
 (segment (start 120.015 80.345) (end 129.94 70.42) (width 0.2) (layer "F.Cu") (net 8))
 (segment (start 120.015 99.85375) (end 120.015 80.345) (width 0.2) (layer "F.Cu") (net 8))
 (segment (start 137.9 68.06) (end 130.12 68.06) (width 0.2) (layer "F.Cu") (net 5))
 (segment (start 130.12 68.06) (end 129.94 67.88) (width 0.2) (layer "F.Cu") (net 5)))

